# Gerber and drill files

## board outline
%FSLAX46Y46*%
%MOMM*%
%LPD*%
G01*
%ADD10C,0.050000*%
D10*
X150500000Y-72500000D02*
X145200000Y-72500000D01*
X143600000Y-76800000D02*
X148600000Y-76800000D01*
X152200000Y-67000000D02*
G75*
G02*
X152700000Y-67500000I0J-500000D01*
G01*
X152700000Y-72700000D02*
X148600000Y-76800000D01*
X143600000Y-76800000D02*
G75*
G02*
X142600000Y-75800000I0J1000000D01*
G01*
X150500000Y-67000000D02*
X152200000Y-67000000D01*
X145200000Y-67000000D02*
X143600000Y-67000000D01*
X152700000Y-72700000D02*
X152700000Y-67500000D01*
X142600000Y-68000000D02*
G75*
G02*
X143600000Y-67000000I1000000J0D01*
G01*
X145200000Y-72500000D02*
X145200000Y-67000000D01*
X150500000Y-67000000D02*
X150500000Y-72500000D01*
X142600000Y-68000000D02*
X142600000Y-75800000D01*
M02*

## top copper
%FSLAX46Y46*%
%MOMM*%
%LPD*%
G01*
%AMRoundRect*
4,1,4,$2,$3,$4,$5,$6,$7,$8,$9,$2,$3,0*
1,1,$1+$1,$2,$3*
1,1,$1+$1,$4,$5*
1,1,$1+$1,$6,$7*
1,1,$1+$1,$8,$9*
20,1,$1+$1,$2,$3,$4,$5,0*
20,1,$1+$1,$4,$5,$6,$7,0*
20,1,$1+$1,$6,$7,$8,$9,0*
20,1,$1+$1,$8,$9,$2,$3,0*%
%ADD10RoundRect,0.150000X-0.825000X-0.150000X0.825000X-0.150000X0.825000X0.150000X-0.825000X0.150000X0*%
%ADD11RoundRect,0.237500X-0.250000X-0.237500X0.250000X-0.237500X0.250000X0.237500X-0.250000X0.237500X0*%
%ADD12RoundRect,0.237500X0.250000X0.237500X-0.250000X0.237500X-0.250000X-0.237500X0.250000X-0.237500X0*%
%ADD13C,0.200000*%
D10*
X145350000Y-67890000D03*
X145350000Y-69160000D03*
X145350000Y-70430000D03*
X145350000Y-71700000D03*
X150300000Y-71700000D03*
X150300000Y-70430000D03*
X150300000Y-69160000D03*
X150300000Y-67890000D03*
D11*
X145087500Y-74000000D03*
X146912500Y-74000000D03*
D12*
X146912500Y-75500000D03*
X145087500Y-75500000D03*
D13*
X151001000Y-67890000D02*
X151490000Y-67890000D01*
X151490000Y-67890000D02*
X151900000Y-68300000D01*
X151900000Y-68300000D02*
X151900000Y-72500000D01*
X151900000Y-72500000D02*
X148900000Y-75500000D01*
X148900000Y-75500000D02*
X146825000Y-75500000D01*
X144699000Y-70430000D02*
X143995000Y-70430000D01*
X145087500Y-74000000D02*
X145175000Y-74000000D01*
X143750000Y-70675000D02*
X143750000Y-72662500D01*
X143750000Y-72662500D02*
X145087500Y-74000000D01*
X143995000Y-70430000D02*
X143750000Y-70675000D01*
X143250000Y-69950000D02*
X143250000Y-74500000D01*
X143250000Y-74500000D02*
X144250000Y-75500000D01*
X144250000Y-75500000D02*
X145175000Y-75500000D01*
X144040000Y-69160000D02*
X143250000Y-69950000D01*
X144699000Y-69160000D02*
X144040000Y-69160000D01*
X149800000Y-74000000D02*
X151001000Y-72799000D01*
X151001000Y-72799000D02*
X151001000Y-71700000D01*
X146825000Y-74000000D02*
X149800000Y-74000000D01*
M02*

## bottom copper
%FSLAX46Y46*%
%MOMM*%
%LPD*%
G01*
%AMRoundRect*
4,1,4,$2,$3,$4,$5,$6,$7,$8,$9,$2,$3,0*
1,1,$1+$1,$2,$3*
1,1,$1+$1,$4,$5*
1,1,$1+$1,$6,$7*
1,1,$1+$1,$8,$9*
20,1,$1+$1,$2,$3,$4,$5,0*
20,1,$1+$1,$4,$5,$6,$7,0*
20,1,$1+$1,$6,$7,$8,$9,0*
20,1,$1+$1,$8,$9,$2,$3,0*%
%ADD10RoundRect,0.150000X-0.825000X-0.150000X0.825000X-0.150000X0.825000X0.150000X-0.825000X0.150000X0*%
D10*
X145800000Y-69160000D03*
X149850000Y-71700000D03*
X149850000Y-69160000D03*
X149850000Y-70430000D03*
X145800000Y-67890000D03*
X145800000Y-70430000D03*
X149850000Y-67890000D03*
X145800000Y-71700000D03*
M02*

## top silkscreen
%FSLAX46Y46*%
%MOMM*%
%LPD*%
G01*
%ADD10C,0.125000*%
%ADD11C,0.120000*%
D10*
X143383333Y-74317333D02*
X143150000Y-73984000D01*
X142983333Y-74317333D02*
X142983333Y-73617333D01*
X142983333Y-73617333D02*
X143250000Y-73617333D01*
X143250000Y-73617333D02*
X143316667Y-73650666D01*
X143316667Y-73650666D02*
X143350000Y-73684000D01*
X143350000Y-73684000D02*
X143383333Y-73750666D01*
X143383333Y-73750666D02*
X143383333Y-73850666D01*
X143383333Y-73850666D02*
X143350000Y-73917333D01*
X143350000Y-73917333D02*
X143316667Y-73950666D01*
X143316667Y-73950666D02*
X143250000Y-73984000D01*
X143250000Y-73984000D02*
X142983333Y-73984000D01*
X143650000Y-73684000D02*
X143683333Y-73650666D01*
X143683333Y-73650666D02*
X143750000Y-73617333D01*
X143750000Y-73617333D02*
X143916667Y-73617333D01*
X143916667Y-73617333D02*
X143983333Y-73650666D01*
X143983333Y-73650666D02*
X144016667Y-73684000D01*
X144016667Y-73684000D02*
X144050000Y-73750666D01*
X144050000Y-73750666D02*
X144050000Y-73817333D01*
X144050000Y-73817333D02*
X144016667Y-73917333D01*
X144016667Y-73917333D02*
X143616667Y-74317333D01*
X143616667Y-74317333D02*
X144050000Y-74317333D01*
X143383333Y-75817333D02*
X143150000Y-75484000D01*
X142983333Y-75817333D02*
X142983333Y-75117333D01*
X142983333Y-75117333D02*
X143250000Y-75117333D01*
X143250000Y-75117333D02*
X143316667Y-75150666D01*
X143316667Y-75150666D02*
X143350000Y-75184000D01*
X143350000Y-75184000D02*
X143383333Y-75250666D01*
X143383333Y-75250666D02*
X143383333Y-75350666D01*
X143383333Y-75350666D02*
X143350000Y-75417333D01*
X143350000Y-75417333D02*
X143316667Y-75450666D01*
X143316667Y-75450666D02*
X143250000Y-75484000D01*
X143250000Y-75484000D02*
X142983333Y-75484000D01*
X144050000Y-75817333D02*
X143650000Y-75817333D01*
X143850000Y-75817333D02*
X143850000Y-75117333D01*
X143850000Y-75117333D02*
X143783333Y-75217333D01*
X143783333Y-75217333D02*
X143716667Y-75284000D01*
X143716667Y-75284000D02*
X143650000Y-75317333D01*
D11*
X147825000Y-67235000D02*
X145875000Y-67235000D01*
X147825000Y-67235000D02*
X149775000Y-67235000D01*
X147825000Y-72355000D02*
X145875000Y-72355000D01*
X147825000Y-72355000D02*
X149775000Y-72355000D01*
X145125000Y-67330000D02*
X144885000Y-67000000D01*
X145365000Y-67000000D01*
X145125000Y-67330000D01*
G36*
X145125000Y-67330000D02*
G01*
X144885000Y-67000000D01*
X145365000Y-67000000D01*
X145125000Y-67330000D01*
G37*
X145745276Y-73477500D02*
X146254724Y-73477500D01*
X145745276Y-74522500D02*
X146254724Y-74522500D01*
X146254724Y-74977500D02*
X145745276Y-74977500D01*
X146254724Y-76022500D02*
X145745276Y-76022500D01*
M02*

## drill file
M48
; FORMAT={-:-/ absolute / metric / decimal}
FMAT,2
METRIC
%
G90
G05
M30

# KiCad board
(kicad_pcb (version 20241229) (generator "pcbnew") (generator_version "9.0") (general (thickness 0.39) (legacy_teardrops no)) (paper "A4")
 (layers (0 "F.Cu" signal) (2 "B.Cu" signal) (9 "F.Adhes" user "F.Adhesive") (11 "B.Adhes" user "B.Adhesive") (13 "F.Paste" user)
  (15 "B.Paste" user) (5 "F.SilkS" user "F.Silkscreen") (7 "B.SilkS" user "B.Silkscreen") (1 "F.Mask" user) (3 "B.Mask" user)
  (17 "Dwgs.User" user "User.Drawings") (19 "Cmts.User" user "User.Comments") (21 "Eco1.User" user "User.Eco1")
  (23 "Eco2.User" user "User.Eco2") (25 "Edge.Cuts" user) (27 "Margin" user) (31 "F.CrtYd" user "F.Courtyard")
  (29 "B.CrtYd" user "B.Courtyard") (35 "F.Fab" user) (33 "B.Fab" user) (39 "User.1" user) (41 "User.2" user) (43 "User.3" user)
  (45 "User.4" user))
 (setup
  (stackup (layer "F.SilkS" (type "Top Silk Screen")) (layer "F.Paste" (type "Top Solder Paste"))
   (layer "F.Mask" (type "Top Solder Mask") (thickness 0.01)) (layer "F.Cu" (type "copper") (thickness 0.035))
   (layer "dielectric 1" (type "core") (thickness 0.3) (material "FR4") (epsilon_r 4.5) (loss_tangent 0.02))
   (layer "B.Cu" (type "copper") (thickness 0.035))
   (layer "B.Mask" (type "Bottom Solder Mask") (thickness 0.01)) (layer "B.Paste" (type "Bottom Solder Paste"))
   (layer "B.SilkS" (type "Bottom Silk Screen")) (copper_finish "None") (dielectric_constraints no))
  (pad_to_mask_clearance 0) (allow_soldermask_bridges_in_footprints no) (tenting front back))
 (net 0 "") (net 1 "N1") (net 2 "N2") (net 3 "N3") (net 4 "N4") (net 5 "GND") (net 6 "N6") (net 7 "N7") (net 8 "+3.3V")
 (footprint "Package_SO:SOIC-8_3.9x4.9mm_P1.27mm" (layer "F.Cu") (at 147.825 69.795)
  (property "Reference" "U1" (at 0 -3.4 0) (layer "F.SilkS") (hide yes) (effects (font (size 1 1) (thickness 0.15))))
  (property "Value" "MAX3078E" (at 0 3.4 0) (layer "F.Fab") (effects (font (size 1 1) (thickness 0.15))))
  (fp_line (start 0 -2.56) (end -1.95 -2.56) (stroke (width 0.12) (type solid)) (layer "F.SilkS"))
  (fp_line (start 0 -2.56) (end 1.95 -2.56) (stroke (width 0.12) (type solid)) (layer "F.SilkS"))
  (fp_line (start 0 2.56) (end -1.95 2.56) (stroke (width 0.12) (type solid)) (layer "F.SilkS"))
  (fp_line (start 0 2.56) (end 1.95 2.56) (stroke (width 0.12) (type solid)) (layer "F.SilkS"))
  (fp_poly (pts (xy -2.7 -2.465) (xy -2.94 -2.795) (xy -2.46 -2.795)) (stroke (width 0.12) (type solid)) (fill yes) (layer "F.SilkS"))
  (pad "1" smd roundrect (at -2.475 -1.905) (size 1.95 0.6) (layers "F.Cu" "F.Mask" "F.Paste") (roundrect_rratio 0.25) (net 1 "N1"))
  (pad "2" smd roundrect (at -2.475 -0.635) (size 1.95 0.6) (layers "F.Cu" "F.Mask" "F.Paste") (roundrect_rratio 0.25) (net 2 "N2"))
  (pad "3" smd roundrect (at -2.475 0.635) (size 1.95 0.6) (layers "F.Cu" "F.Mask" "F.Paste") (roundrect_rratio 0.25) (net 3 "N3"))
  (pad "4" smd roundrect (at -2.475 1.905) (size 1.95 0.6) (layers "F.Cu" "F.Mask" "F.Paste") (roundrect_rratio 0.25) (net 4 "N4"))
  (pad "5" smd roundrect (at 2.475 1.905) (size 1.95 0.6) (layers "F.Cu" "F.Mask" "F.Paste") (roundrect_rratio 0.25) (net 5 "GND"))
  (pad "6" smd roundrect (at 2.475 0.635) (size 1.95 0.6) (layers "F.Cu" "F.Mask" "F.Paste") (roundrect_rratio 0.25) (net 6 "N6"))
  (pad "7" smd roundrect (at 2.475 -0.635) (size 1.95 0.6) (layers "F.Cu" "F.Mask" "F.Paste") (roundrect_rratio 0.25) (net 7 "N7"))
  (pad "8" smd roundrect (at 2.475 -1.905) (size 1.95 0.6) (layers "F.Cu" "F.Mask" "F.Paste") (roundrect_rratio 0.25) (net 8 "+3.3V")))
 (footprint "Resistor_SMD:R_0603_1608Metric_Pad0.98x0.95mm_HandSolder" (layer "F.Cu") (at 146 74)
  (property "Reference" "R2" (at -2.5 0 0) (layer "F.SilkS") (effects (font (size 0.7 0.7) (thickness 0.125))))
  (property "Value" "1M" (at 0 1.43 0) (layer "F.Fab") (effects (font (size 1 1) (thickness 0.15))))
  (fp_line (start -0.254724 -0.5225) (end 0.254724 -0.5225) (stroke (width 0.12) (type solid)) (layer "F.SilkS"))
  (fp_line (start -0.254724 0.5225) (end 0.254724 0.5225) (stroke (width 0.12) (type solid)) (layer "F.SilkS"))
  (pad "1" smd roundrect (at -0.9125 0) (size 0.975 0.95) (layers "F.Cu" "F.Mask" "F.Paste") (roundrect_rratio 0.25) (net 3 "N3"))
  (pad "2" smd roundrect (at 0.9125 0) (size 0.975 0.95) (layers "F.Cu" "F.Mask" "F.Paste") (roundrect_rratio 0.25) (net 5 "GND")))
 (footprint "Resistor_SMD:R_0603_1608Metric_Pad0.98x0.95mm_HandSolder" (layer "F.Cu") (at 146 75.5 180)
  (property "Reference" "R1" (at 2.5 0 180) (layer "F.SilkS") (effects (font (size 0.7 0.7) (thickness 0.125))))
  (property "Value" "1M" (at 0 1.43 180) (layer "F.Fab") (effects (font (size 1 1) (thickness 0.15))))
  (fp_line (start -0.254724 0.5225) (end 0.254724 0.5225) (stroke (width 0.12) (type solid)) (layer "F.SilkS"))
  (fp_line (start -0.254724 -0.5225) (end 0.254724 -0.5225) (stroke (width 0.12) (type solid)) (layer "F.SilkS"))
  (pad "1" smd roundrect (at -0.9125 0 180) (size 0.975 0.95) (layers "F.Cu" "F.Mask" "F.Paste") (roundrect_rratio 0.25) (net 8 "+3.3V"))
  (pad "2" smd roundrect (at 0.9125 0 180) (size 0.975 0.95) (layers "F.Cu" "F.Mask" "F.Paste") (roundrect_rratio 0.25) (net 2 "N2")))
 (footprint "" (layer "B.Cu") (at 145.8 69.16)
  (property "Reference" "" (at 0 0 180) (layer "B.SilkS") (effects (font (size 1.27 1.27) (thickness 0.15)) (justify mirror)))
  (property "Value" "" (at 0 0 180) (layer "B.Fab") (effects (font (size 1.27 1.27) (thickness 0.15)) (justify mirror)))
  (pad "2" smd roundrect (at 0 0) (size 1.95 0.6) (layers "B.Cu" "B.Mask" "B.Paste") (roundrect_rratio 0.25) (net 2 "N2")))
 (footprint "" (layer "B.Cu") (at 149.85 71.7)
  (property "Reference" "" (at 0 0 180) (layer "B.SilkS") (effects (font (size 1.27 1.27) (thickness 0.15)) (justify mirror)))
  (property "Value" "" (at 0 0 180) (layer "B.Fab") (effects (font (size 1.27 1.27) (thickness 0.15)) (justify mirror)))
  (pad "5" smd roundrect (at 0 0) (size 1.95 0.6) (layers "B.Cu" "B.Mask" "B.Paste") (roundrect_rratio 0.25) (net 5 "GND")))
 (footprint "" (layer "B.Cu") (at 149.85 69.16)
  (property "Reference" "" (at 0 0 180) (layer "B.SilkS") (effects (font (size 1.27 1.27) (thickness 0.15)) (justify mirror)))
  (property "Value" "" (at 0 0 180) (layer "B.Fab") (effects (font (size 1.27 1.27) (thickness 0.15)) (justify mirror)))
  (pad "7" smd roundrect (at 0 0) (size 1.95 0.6) (layers "B.Cu" "B.Mask" "B.Paste") (roundrect_rratio 0.25) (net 7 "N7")))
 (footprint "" (layer "B.Cu") (at 149.85 70.43)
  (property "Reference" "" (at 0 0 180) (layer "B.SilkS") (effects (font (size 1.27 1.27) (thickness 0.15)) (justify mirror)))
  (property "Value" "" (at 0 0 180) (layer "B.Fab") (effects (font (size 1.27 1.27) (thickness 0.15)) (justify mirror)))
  (pad "6" smd roundrect (at 0 0) (size 1.95 0.6) (layers "B.Cu" "B.Mask" "B.Paste") (roundrect_rratio 0.25) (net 6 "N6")))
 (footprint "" (layer "B.Cu") (at 145.8 67.89)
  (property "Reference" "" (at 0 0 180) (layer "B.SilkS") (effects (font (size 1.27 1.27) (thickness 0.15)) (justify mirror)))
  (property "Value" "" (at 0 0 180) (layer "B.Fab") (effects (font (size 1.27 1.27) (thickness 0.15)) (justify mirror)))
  (pad "1" smd roundrect (at 0 0) (size 1.95 0.6) (layers "B.Cu" "B.Mask" "B.Paste") (roundrect_rratio 0.25) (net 1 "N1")))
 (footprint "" (layer "B.Cu") (at 145.8 70.43)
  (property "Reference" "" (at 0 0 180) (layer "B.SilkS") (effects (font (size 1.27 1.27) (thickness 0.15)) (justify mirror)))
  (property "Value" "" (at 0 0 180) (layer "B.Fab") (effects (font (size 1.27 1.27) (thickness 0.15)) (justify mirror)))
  (pad "3" smd roundrect (at 0 0) (size 1.95 0.6) (layers "B.Cu" "B.Mask" "B.Paste") (roundrect_rratio 0.25) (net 3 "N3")))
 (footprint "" (layer "B.Cu") (at 149.85 67.89)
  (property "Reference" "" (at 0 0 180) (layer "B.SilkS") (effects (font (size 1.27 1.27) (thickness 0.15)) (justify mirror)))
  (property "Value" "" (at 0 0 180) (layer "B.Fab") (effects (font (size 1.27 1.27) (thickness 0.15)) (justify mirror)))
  (pad "8" smd roundrect (at 0 0) (size 1.95 0.6) (layers "B.Cu" "B.Mask" "B.Paste") (roundrect_rratio 0.25) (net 8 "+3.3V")))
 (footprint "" (layer "B.Cu") (at 145.8 71.7)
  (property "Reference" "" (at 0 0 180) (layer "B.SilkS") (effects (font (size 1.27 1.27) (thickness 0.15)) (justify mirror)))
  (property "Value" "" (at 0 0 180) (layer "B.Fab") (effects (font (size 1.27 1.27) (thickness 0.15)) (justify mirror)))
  (pad "4" smd roundrect (at 0 0) (size 1.95 0.6) (layers "B.Cu" "B.Mask" "B.Paste") (roundrect_rratio 0.25) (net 4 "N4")))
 (gr_line (start 150.5 72.5) (end 145.2 72.5) (stroke (width 0.05) (type default)) (layer "Edge.Cuts"))
 (gr_line (start 143.6 76.8) (end 148.6 76.8) (stroke (width 0.05) (type default)) (layer "Edge.Cuts"))
 (gr_arc (start 152.2 67) (mid 152.553553 67.146447) (end 152.7 67.5) (stroke (width 0.05) (type default)) (layer "Edge.Cuts"))
 (gr_line (start 152.7 72.7) (end 148.6 76.8) (stroke (width 0.05) (type solid)) (layer "Edge.Cuts"))
 (gr_arc (start 143.6 76.8) (mid 142.892893 76.507107) (end 142.6 75.8) (stroke (width 0.05) (type default)) (layer "Edge.Cuts"))
 (gr_line (start 150.5 67) (end 152.2 67) (stroke (width 0.05) (type default)) (layer "Edge.Cuts"))
 (gr_line (start 145.2 67) (end 143.6 67) (stroke (width 0.05) (type default)) (layer "Edge.Cuts"))
 (gr_line (start 152.7 72.7) (end 152.7 67.5) (stroke (width 0.05) (type default)) (layer "Edge.Cuts"))
 (gr_arc (start 142.6 68) (mid 142.892893 67.292893) (end 143.6 67) (stroke (width 0.05) (type default)) (layer "Edge.Cuts"))
 (gr_line (start 145.2 72.5) (end 145.2 67) (stroke (width 0.05) (type default)) (layer "Edge.Cuts"))
 (gr_line (start 150.5 67) (end 150.5 72.5) (stroke (width 0.05) (type default)) (layer "Edge.Cuts"))
 (gr_line (start 142.6 68) (end 142.6 75.8) (stroke (width 0.05) (type default)) (layer "Edge.Cuts"))
 (segment (start 151.001 67.89) (end 151.49 67.89) (width 0.2) (layer "F.Cu") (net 8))
 (segment (start 151.49 67.89) (end 151.9 68.3) (width 0.2) (layer "F.Cu") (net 8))
 (segment (start 151.9 68.3) (end 151.9 72.5) (width 0.2) (layer "F.Cu") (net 8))
 (segment (start 151.9 72.5) (end 148.9 75.5) (width 0.2) (layer "F.Cu") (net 8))
 (segment (start 148.9 75.5) (end 146.825 75.5) (width 0.2) (layer "F.Cu") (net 8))
 (segment (start 144.699 70.43) (end 143.995 70.43) (width 0.2) (layer "F.Cu") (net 3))
 (segment (start 145.0875 74) (end 145.175 74) (width 0.2) (layer "F.Cu") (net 3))
 (segment (start 143.75 70.675) (end 143.75 72.6625) (width 0.2) (layer "F.Cu") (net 3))
 (segment (start 143.75 72.6625) (end 145.0875 74) (width 0.2) (layer "F.Cu") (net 3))
 (segment (start 143.995 70.43) (end 143.75 70.675) (width 0.2) (layer "F.Cu") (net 3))
 (segment (start 143.25 69.95) (end 143.25 74.5) (width 0.2) (layer "F.Cu") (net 2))
 (segment (start 143.25 74.5) (end 144.25 75.5) (width 0.2) (layer "F.Cu") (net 2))
 (segment (start 144.25 75.5) (end 145.175 75.5) (width 0.2) (layer "F.Cu") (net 2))
 (segment (start 144.04 69.16) (end 143.25 69.95) (width 0.2) (layer "F.Cu") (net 2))
 (segment (start 144.699 69.16) (end 144.04 69.16) (width 0.2) (layer "F.Cu") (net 2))
 (segment (start 149.8 74) (end 151.001 72.799) (width 0.2) (layer "F.Cu") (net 5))
 (segment (start 151.001 72.799) (end 151.001 71.7) (width 0.2) (layer "F.Cu") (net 5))
 (segment (start 146.825 74) (end 149.8 74) (width 0.2) (layer "F.Cu") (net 5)))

